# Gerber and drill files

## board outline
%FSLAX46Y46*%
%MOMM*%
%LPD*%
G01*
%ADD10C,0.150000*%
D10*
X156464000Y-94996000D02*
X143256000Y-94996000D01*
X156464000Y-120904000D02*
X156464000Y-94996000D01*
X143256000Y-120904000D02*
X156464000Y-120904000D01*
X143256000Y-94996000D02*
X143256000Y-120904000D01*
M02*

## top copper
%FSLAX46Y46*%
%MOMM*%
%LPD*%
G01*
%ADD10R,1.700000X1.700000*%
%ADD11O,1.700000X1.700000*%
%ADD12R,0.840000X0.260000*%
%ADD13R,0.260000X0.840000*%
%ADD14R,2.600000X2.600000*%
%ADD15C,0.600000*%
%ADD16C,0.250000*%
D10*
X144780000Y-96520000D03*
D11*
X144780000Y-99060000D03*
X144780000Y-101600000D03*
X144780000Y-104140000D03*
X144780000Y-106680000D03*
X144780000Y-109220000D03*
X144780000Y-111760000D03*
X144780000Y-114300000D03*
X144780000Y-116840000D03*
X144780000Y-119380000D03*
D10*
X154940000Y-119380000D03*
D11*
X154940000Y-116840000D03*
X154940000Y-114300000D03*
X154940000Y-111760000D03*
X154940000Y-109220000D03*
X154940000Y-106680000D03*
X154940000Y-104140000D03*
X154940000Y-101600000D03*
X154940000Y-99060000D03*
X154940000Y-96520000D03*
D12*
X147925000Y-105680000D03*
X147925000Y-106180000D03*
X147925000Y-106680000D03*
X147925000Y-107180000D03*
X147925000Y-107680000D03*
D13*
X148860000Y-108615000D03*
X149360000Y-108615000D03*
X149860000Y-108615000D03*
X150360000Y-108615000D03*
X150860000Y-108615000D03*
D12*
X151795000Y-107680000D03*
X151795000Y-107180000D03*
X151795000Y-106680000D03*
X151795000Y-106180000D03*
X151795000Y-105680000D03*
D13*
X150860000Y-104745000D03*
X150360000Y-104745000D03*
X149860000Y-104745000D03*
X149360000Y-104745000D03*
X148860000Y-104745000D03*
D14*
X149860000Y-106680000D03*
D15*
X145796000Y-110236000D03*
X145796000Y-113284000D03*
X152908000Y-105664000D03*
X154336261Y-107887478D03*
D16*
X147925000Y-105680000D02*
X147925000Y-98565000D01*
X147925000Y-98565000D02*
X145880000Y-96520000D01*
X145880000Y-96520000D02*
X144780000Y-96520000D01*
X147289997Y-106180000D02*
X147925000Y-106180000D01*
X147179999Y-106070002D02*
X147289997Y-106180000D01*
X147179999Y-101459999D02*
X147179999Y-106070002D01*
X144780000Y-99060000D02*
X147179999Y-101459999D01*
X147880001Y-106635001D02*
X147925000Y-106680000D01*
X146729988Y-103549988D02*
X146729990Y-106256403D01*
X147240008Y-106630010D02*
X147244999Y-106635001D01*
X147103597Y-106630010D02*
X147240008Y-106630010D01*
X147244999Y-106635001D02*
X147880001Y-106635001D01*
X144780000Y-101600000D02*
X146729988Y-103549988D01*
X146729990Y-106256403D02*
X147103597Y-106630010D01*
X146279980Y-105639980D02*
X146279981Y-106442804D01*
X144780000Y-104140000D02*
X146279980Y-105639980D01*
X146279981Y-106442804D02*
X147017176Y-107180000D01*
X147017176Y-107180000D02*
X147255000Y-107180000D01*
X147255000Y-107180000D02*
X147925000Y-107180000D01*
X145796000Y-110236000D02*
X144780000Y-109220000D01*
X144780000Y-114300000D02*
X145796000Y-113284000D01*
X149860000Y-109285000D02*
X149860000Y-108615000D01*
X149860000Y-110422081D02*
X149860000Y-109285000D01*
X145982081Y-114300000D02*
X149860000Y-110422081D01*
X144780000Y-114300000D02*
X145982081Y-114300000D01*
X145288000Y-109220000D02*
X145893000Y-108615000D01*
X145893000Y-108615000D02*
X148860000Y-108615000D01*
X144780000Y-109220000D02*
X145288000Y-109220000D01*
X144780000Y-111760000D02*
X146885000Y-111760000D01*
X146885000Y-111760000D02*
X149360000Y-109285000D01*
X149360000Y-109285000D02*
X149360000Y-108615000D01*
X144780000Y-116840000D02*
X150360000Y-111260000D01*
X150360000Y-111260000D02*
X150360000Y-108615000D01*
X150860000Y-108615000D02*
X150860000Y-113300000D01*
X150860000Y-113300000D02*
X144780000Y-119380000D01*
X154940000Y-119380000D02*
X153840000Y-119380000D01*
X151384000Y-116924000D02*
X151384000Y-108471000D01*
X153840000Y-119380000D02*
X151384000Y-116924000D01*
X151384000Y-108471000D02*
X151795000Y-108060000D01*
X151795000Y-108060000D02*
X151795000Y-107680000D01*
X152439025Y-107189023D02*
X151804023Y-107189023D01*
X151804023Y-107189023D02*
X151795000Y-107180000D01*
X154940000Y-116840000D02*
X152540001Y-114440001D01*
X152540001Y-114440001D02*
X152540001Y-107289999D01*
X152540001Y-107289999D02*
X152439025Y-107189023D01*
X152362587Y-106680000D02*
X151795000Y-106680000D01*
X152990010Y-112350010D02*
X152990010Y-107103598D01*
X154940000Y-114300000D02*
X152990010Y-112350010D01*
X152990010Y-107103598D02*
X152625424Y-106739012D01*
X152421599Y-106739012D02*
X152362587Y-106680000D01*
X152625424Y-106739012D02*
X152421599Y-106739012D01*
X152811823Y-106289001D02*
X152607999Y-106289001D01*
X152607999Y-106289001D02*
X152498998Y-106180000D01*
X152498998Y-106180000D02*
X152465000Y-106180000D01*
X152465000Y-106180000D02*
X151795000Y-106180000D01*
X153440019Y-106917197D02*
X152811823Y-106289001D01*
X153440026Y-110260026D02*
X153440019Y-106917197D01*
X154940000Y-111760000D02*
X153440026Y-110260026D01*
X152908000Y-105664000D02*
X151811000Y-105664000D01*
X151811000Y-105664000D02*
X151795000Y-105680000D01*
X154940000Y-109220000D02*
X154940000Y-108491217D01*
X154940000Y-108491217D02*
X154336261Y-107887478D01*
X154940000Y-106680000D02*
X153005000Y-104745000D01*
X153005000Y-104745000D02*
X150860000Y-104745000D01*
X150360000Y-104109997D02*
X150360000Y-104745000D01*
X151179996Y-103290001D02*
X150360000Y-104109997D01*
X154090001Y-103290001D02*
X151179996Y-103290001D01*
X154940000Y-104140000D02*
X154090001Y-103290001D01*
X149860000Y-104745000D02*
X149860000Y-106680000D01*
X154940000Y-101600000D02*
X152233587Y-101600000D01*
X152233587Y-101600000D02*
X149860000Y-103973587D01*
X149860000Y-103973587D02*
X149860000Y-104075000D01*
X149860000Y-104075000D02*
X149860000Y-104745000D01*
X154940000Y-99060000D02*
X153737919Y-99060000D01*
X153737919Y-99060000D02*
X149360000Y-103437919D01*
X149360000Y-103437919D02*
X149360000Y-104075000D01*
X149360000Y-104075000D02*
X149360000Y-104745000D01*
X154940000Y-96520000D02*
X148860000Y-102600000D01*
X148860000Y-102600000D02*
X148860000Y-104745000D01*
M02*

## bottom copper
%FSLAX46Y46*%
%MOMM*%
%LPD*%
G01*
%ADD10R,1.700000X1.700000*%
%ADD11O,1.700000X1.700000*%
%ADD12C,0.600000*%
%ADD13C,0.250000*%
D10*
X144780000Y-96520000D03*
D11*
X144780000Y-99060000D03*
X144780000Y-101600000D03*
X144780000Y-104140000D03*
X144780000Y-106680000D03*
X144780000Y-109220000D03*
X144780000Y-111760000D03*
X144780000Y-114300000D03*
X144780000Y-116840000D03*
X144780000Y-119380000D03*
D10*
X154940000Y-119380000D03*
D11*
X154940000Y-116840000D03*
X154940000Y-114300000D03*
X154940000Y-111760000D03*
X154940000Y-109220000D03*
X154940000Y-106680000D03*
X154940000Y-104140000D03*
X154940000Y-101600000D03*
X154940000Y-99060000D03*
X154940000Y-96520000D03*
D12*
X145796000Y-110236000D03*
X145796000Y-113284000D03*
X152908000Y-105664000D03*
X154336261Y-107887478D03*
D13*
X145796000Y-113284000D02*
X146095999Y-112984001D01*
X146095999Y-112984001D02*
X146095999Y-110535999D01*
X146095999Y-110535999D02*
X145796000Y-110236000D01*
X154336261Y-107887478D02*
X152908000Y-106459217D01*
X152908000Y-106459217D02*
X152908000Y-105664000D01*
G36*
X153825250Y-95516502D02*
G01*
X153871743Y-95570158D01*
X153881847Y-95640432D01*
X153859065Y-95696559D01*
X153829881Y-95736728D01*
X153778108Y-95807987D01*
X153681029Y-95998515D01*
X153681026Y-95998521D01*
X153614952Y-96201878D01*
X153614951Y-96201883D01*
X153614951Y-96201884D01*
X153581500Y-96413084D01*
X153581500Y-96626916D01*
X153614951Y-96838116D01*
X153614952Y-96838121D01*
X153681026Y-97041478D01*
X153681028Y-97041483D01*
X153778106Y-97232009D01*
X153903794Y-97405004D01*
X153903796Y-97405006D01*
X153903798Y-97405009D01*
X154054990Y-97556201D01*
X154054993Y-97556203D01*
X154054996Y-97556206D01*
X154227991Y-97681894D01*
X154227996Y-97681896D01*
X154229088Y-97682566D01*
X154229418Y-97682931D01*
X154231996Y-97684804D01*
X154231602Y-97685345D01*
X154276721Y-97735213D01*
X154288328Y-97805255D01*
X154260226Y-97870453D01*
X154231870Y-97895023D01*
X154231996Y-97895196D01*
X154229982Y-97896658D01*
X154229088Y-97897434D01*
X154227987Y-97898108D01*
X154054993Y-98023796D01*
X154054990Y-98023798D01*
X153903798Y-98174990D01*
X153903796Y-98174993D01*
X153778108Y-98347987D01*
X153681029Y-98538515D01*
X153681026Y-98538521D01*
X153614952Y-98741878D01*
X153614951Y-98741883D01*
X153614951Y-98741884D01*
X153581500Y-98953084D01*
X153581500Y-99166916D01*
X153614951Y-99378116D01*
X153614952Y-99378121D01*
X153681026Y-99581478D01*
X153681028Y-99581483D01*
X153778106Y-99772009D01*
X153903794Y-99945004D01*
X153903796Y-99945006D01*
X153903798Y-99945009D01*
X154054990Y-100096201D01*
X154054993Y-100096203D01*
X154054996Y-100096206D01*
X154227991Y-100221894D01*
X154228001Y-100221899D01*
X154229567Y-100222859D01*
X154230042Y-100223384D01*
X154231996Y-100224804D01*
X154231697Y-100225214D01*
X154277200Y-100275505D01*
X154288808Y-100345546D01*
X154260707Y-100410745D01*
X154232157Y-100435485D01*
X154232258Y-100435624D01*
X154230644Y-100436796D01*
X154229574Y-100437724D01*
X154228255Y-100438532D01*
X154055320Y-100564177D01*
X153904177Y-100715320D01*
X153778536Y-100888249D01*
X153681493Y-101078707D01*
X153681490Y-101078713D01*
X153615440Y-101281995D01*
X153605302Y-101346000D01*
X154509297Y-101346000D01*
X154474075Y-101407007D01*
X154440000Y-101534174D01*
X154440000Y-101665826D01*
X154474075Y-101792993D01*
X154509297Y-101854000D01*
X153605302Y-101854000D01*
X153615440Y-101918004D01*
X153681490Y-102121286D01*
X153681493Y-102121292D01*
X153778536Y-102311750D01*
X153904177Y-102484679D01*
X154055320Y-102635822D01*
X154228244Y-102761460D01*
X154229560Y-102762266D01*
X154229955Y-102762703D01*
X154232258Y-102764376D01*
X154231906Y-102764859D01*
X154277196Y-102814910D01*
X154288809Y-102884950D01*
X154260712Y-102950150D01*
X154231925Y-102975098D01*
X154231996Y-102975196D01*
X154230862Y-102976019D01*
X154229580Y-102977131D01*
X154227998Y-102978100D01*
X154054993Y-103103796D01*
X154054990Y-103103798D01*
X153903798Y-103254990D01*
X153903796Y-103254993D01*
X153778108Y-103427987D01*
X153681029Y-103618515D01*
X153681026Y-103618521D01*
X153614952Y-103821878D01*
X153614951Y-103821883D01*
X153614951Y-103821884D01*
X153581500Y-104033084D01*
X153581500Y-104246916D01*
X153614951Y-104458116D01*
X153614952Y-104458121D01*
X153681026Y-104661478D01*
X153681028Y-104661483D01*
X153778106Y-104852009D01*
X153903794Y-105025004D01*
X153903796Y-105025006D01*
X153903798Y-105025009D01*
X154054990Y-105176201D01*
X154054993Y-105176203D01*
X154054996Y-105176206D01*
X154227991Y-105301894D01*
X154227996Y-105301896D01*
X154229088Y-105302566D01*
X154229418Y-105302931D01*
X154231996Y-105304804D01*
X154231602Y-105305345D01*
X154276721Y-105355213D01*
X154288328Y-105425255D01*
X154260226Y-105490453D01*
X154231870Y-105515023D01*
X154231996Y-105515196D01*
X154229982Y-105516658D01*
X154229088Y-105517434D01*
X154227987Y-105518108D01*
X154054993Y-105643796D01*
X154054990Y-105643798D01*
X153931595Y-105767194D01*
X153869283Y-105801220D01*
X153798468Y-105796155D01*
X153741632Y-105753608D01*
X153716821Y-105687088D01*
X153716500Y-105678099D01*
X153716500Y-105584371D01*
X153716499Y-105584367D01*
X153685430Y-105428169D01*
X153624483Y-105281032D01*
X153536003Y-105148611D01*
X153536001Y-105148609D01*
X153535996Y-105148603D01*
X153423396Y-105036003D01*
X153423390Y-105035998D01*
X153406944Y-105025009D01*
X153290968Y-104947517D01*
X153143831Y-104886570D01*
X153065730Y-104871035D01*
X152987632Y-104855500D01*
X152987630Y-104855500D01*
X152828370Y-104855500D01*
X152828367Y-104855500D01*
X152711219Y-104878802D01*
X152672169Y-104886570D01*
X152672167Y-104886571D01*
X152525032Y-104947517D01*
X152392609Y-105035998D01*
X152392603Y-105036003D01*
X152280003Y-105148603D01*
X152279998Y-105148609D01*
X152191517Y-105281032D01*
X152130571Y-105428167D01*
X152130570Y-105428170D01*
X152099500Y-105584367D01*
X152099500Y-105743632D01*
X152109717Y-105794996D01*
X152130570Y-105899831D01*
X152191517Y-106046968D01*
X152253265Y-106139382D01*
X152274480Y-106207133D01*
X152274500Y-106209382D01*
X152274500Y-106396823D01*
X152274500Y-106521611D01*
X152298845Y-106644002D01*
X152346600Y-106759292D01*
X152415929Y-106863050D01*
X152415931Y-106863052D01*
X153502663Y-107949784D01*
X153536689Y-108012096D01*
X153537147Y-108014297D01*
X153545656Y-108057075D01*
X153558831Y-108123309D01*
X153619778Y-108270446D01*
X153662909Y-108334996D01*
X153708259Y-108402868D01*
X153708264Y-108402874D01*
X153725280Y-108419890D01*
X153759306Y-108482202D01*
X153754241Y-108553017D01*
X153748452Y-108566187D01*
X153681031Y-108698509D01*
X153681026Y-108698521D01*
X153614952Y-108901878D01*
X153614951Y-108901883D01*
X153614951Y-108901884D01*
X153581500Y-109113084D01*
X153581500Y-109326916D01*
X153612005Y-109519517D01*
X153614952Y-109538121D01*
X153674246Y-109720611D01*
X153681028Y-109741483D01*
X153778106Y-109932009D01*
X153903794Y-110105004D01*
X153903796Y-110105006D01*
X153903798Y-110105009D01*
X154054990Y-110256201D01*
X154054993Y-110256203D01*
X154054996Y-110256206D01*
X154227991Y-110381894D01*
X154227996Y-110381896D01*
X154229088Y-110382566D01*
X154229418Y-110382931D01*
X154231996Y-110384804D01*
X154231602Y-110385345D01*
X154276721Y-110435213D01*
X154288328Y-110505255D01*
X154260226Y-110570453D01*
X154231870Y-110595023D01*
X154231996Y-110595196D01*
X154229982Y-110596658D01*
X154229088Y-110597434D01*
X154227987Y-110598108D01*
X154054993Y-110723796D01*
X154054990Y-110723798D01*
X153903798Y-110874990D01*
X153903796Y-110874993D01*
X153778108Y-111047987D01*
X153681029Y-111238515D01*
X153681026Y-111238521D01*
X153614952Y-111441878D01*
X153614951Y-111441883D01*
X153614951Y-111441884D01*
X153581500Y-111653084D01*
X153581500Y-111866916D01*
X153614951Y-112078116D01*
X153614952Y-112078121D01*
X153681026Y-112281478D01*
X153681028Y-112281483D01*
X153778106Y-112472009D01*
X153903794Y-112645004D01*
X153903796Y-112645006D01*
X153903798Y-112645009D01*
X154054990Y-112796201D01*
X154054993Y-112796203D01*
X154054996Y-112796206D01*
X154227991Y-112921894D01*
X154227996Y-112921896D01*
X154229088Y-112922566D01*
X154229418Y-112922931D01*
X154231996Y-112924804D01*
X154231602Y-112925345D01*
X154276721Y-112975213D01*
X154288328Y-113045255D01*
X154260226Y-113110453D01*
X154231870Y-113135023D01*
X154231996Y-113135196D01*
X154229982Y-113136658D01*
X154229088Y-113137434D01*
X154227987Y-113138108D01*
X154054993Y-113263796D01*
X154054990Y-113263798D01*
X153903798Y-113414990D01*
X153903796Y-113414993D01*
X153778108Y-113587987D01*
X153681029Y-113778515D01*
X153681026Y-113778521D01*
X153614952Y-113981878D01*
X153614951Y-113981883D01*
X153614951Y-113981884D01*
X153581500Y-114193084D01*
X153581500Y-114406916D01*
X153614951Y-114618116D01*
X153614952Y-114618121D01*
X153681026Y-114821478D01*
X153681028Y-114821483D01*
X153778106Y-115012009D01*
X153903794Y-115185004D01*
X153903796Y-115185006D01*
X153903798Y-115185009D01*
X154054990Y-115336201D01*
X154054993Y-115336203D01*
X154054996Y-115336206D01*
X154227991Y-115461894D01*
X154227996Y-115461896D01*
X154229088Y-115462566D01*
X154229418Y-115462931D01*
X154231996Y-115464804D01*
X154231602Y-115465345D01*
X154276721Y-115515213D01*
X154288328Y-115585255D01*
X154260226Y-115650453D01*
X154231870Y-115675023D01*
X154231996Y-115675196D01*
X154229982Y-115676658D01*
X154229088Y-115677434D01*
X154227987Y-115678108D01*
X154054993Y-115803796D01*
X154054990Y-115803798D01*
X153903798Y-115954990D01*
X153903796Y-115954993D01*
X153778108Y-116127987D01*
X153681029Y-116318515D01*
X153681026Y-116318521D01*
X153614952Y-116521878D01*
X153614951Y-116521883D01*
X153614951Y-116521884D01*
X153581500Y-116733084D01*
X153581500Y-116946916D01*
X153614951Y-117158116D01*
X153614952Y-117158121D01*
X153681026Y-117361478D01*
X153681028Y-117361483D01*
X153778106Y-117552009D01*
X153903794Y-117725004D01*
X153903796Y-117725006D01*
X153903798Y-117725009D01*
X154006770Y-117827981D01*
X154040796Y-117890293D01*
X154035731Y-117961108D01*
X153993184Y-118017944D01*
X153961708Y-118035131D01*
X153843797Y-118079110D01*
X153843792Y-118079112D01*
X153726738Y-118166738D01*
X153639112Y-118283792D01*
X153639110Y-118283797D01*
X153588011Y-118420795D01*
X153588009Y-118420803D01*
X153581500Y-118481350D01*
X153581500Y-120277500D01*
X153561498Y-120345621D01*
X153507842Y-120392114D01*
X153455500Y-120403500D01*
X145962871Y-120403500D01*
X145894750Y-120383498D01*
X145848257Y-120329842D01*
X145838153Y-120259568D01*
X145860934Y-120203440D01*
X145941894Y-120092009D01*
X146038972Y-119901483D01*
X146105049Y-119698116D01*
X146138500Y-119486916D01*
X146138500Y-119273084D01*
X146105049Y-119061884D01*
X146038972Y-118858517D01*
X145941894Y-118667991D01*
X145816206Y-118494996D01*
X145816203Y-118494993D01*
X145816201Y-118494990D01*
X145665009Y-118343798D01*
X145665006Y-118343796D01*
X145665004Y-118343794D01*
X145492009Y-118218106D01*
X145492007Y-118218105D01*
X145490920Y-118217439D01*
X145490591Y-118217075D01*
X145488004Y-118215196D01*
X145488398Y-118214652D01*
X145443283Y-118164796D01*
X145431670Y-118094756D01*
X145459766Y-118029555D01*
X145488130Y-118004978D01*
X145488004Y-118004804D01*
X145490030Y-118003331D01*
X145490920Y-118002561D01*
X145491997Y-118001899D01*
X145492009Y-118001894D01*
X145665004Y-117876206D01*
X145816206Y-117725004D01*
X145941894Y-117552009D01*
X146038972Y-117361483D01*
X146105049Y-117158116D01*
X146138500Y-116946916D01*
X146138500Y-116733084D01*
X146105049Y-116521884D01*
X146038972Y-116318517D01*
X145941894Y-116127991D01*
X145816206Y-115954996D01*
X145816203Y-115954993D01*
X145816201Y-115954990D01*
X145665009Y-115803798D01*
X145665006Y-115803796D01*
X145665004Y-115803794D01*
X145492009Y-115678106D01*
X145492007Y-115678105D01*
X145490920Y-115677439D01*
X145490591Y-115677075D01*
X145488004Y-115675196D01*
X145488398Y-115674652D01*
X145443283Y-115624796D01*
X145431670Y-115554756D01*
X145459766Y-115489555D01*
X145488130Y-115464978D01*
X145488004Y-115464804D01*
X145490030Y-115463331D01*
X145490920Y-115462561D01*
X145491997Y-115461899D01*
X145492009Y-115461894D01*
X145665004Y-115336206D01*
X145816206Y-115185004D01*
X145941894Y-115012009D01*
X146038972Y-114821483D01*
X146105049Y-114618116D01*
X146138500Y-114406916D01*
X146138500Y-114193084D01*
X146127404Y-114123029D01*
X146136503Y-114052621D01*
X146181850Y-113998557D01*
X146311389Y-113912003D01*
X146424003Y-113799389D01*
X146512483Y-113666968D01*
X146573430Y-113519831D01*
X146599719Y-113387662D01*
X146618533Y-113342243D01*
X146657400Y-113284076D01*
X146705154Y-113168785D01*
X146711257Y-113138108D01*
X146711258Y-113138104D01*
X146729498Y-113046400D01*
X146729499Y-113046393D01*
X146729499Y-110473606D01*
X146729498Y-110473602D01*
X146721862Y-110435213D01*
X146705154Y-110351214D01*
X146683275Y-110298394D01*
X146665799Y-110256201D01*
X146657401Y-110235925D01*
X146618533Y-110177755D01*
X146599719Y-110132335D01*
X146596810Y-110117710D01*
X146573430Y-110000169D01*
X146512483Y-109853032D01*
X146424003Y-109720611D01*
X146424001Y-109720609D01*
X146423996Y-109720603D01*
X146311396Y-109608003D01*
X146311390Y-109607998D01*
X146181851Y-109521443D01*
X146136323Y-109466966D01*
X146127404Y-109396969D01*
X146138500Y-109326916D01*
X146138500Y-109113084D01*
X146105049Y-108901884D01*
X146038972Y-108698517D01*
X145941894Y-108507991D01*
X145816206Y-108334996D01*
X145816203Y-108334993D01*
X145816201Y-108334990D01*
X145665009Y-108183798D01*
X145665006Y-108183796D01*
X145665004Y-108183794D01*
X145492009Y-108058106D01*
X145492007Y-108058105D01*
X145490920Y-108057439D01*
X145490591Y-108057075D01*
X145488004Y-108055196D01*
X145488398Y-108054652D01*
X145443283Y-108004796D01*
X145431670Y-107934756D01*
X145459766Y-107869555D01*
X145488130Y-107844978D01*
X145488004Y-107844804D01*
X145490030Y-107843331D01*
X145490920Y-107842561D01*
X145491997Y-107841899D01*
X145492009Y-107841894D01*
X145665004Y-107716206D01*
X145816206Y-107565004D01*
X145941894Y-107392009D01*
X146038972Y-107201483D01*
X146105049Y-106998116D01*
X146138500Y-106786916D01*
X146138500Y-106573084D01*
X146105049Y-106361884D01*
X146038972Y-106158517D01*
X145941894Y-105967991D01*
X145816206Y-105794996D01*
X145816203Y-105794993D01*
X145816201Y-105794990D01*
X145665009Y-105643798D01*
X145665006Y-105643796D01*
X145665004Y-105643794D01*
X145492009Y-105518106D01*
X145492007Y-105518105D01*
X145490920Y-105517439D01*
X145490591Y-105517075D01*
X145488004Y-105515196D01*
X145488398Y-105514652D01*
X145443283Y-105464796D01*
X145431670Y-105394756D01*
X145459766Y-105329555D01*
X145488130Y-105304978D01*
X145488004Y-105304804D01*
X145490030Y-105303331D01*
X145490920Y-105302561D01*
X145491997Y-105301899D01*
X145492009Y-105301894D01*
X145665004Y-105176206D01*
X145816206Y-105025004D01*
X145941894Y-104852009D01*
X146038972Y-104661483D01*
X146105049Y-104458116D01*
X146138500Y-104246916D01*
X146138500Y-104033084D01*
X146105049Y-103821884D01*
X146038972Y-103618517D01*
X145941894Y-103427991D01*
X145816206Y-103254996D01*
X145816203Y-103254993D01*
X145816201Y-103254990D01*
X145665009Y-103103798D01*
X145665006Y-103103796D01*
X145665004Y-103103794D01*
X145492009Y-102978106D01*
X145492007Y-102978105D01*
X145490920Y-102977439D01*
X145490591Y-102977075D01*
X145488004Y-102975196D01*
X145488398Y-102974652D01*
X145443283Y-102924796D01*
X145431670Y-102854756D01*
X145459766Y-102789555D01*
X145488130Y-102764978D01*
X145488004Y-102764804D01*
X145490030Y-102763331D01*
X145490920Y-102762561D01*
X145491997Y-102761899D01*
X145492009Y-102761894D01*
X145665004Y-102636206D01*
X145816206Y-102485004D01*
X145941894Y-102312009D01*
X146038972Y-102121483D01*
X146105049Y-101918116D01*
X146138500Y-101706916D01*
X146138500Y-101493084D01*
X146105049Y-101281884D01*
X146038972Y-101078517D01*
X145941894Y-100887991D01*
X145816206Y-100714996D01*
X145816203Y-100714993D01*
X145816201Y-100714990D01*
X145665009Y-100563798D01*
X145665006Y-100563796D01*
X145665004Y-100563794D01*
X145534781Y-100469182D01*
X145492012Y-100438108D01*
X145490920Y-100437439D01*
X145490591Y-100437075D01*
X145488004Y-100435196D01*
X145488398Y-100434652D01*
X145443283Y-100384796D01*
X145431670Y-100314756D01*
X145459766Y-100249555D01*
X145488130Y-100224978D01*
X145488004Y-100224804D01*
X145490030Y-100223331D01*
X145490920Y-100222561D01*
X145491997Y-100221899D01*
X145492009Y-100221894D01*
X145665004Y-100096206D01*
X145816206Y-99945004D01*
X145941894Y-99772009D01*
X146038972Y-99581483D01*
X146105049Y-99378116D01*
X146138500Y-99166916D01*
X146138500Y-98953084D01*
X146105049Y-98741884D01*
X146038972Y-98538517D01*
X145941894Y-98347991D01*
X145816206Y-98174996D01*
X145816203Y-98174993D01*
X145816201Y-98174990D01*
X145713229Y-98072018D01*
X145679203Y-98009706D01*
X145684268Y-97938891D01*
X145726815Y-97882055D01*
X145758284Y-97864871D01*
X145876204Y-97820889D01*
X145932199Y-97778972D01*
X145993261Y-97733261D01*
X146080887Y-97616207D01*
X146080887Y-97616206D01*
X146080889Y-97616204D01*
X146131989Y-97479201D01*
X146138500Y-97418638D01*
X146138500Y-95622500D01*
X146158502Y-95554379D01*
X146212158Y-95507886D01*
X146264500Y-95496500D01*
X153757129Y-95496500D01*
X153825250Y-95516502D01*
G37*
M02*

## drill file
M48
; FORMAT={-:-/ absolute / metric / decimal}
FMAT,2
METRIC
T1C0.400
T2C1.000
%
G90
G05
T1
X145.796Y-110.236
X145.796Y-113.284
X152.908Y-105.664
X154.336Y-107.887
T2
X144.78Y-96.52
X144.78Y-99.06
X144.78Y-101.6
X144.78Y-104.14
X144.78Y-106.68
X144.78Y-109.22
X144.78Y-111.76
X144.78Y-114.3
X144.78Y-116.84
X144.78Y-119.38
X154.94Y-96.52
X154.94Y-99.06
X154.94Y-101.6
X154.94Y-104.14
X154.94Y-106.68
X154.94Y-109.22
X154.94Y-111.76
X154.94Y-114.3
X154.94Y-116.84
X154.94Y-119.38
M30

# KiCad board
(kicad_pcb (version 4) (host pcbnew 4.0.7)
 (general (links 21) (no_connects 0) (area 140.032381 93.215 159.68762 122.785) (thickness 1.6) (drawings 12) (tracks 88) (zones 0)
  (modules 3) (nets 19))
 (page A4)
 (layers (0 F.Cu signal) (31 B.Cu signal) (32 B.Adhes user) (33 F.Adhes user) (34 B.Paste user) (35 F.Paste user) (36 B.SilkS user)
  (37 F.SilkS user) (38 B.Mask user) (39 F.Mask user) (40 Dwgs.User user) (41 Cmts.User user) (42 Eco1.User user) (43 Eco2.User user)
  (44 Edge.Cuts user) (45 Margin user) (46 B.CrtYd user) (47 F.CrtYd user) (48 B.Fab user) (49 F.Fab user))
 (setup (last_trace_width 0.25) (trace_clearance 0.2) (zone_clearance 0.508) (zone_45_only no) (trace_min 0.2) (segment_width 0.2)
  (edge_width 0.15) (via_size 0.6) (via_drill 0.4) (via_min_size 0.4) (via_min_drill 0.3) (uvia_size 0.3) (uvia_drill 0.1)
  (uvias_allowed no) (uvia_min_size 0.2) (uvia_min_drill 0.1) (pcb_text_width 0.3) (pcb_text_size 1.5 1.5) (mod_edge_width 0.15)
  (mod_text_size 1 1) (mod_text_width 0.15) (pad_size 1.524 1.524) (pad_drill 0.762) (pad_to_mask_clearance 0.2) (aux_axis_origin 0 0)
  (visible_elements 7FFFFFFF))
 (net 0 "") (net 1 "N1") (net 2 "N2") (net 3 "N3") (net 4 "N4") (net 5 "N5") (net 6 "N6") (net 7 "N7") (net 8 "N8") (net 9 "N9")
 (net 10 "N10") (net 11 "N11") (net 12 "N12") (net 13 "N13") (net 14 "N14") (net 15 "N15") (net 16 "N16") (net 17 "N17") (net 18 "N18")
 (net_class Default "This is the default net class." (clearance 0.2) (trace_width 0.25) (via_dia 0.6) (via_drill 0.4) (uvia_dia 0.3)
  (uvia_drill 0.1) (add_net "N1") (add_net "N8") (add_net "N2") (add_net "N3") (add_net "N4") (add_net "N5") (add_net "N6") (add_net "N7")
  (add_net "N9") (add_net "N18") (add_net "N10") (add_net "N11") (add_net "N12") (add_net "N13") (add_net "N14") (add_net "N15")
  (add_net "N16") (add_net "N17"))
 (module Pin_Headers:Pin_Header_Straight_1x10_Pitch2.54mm (layer F.Cu) (at 144.78 96.52)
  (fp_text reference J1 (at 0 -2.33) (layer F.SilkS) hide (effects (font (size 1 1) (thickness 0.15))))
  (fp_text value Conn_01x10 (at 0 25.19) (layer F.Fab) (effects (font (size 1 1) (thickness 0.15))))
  (pad 1 thru_hole rect (at 0 0) (size 1.7 1.7) (drill 1) (layers *.Cu *.Mask) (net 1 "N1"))
  (pad 2 thru_hole oval (at 0 2.54) (size 1.7 1.7) (drill 1) (layers *.Cu *.Mask) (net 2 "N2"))
  (pad 3 thru_hole oval (at 0 5.08) (size 1.7 1.7) (drill 1) (layers *.Cu *.Mask) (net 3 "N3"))
  (pad 4 thru_hole oval (at 0 7.62) (size 1.7 1.7) (drill 1) (layers *.Cu *.Mask) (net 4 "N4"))
  (pad 5 thru_hole oval (at 0 10.16) (size 1.7 1.7) (drill 1) (layers *.Cu *.Mask))
  (pad 6 thru_hole oval (at 0 12.7) (size 1.7 1.7) (drill 1) (layers *.Cu *.Mask) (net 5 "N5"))
  (pad 7 thru_hole oval (at 0 15.24) (size 1.7 1.7) (drill 1) (layers *.Cu *.Mask) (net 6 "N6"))
  (pad 8 thru_hole oval (at 0 17.78) (size 1.7 1.7) (drill 1) (layers *.Cu *.Mask) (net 5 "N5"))
  (pad 9 thru_hole oval (at 0 20.32) (size 1.7 1.7) (drill 1) (layers *.Cu *.Mask) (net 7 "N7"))
  (pad 10 thru_hole oval (at 0 22.86) (size 1.7 1.7) (drill 1) (layers *.Cu *.Mask) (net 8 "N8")))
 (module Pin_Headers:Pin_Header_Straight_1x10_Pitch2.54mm (layer F.Cu) (at 154.94 119.38 180)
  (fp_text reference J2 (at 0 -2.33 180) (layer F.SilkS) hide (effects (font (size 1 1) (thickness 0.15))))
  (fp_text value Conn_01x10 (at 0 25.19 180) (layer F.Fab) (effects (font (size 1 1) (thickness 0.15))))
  (pad 1 thru_hole rect (at 0 0 180) (size 1.7 1.7) (drill 1) (layers *.Cu *.Mask) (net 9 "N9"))
  (pad 2 thru_hole oval (at 0 2.54 180) (size 1.7 1.7) (drill 1) (layers *.Cu *.Mask) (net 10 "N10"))
  (pad 3 thru_hole oval (at 0 5.08 180) (size 1.7 1.7) (drill 1) (layers *.Cu *.Mask) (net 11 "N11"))
  (pad 4 thru_hole oval (at 0 7.62 180) (size 1.7 1.7) (drill 1) (layers *.Cu *.Mask) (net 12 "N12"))
  (pad 5 thru_hole oval (at 0 10.16 180) (size 1.7 1.7) (drill 1) (layers *.Cu *.Mask) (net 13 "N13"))
  (pad 6 thru_hole oval (at 0 12.7 180) (size 1.7 1.7) (drill 1) (layers *.Cu *.Mask) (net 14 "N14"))
  (pad 7 thru_hole oval (at 0 15.24 180) (size 1.7 1.7) (drill 1) (layers *.Cu *.Mask) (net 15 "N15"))
  (pad 8 thru_hole oval (at 0 17.78 180) (size 1.7 1.7) (drill 1) (layers *.Cu *.Mask) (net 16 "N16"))
  (pad 9 thru_hole oval (at 0 20.32 180) (size 1.7 1.7) (drill 1) (layers *.Cu *.Mask) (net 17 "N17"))
  (pad 10 thru_hole oval (at 0 22.86 180) (size 1.7 1.7) (drill 1) (layers *.Cu *.Mask) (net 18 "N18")))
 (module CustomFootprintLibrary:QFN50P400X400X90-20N (layer F.Cu) (at 149.86 106.68)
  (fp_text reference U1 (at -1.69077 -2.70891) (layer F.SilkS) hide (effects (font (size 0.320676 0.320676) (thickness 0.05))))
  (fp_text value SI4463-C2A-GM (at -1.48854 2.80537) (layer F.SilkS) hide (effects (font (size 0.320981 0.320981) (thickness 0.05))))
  (pad 1 smd rect (at -1.935 -1 90) (size 0.26 0.84) (layers F.Cu F.Paste F.Mask) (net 1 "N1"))
  (pad 2 smd rect (at -1.935 -0.5 90) (size 0.26 0.84) (layers F.Cu F.Paste F.Mask) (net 2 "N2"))
  (pad 3 smd rect (at -1.935 0 90) (size 0.26 0.84) (layers F.Cu F.Paste F.Mask) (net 3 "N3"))
  (pad 4 smd rect (at -1.935 0.5 90) (size 0.26 0.84) (layers F.Cu F.Paste F.Mask) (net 4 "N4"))
  (pad 5 smd rect (at -1.935 1 90) (size 0.26 0.84) (layers F.Cu F.Paste F.Mask))
  (pad 6 smd rect (at -1 1.935 180) (size 0.26 0.84) (layers F.Cu F.Paste F.Mask) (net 5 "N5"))
  (pad 7 smd rect (at -0.5 1.935 180) (size 0.26 0.84) (layers F.Cu F.Paste F.Mask) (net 6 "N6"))
  (pad 8 smd rect (at 0 1.935 180) (size 0.26 0.84) (layers F.Cu F.Paste F.Mask) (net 5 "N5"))
  (pad 9 smd rect (at 0.5 1.935 180) (size 0.26 0.84) (layers F.Cu F.Paste F.Mask) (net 7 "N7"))
  (pad 10 smd rect (at 1 1.935 180) (size 0.26 0.84) (layers F.Cu F.Paste F.Mask) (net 8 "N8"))
  (pad 11 smd rect (at 1.935 1 270) (size 0.26 0.84) (layers F.Cu F.Paste F.Mask) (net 9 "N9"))
  (pad 12 smd rect (at 1.935 0.5 270) (size 0.26 0.84) (layers F.Cu F.Paste F.Mask) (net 10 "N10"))
  (pad 13 smd rect (at 1.935 0 270) (size 0.26 0.84) (layers F.Cu F.Paste F.Mask) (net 11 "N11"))
  (pad 14 smd rect (at 1.935 -0.5 270) (size 0.26 0.84) (layers F.Cu F.Paste F.Mask) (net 12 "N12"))
  (pad 15 smd rect (at 1.935 -1 270) (size 0.26 0.84) (layers F.Cu F.Paste F.Mask) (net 13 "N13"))
  (pad 16 smd rect (at 1 -1.935) (size 0.26 0.84) (layers F.Cu F.Paste F.Mask) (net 14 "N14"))
  (pad 17 smd rect (at 0.5 -1.935) (size 0.26 0.84) (layers F.Cu F.Paste F.Mask) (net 15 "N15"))
  (pad 18 smd rect (at 0 -1.935) (size 0.26 0.84) (layers F.Cu F.Paste F.Mask) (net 16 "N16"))
  (pad 19 smd rect (at -0.5 -1.935) (size 0.26 0.84) (layers F.Cu F.Paste F.Mask) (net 17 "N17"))
  (pad 20 smd rect (at -1 -1.935) (size 0.26 0.84) (layers F.Cu F.Paste F.Mask) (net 18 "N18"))
  (pad 21 smd rect (at 0 0) (size 2.6 2.6) (layers F.Cu F.Paste F.Mask) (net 16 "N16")))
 (gr_line (start 156.464 94.996) (end 143.256 94.996) (layer Edge.Cuts) (width 0.15))
 (gr_line (start 156.464 120.904) (end 156.464 94.996) (layer Edge.Cuts) (width 0.15))
 (gr_line (start 143.256 120.904) (end 156.464 120.904) (layer Edge.Cuts) (width 0.15))
 (gr_line (start 143.256 94.996) (end 143.256 120.904) (layer Edge.Cuts) (width 0.15))
 (segment (start 147.925 105.68) (end 147.925 98.565) (width 0.25) (layer F.Cu) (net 1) (status 10))
 (segment (start 147.925 98.565) (end 145.88 96.52) (width 0.25) (layer F.Cu) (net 1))
 (segment (start 145.88 96.52) (end 144.78 96.52) (width 0.25) (layer F.Cu) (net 1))
 (segment (start 147.289997 106.18) (end 147.925 106.18) (width 0.25) (layer F.Cu) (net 2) (status 20))
 (segment (start 147.179999 106.070002) (end 147.289997 106.18) (width 0.25) (layer F.Cu) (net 2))
 (segment (start 147.179999 101.459999) (end 147.179999 106.070002) (width 0.25) (layer F.Cu) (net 2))
 (segment (start 144.78 99.06) (end 147.179999 101.459999) (width 0.25) (layer F.Cu) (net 2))
 (segment (start 147.880001 106.635001) (end 147.925 106.68) (width 0.25) (layer F.Cu) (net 3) (status 30))
 (segment (start 146.729988 103.549988) (end 146.72999 106.256403) (width 0.25) (layer F.Cu) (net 3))
 (segment (start 147.240008 106.63001) (end 147.244999 106.635001) (width 0.25) (layer F.Cu) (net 3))
 (segment (start 147.103597 106.63001) (end 147.240008 106.63001) (width 0.25) (layer F.Cu) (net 3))
 (segment (start 147.244999 106.635001) (end 147.880001 106.635001) (width 0.25) (layer F.Cu) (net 3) (status 20))
 (segment (start 144.78 101.6) (end 146.729988 103.549988) (width 0.25) (layer F.Cu) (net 3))
 (segment (start 146.72999 106.256403) (end 147.103597 106.63001) (width 0.25) (layer F.Cu) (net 3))
 (segment (start 146.27998 105.63998) (end 146.279981 106.442804) (width 0.25) (layer F.Cu) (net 4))
 (segment (start 144.78 104.14) (end 146.27998 105.63998) (width 0.25) (layer F.Cu) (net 4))
 (segment (start 146.279981 106.442804) (end 147.017176 107.18) (width 0.25) (layer F.Cu) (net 4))
 (segment (start 147.017176 107.18) (end 147.255 107.18) (width 0.25) (layer F.Cu) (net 4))
 (segment (start 147.255 107.18) (end 147.925 107.18) (width 0.25) (layer F.Cu) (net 4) (status 20))
 (segment (start 145.796 110.236) (end 144.78 109.22) (width 0.25) (layer F.Cu) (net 5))
 (segment (start 145.796 113.284) (end 146.095999 112.984001) (width 0.25) (layer B.Cu) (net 5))
 (segment (start 146.095999 112.984001) (end 146.095999 110.535999) (width 0.25) (layer B.Cu) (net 5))
 (segment (start 146.095999 110.535999) (end 145.796 110.236) (width 0.25) (layer B.Cu) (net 5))
 (via (at 145.796 110.236) (size 0.6) (drill 0.4) (layers F.Cu B.Cu) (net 5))
 (segment (start 144.78 114.3) (end 145.796 113.284) (width 0.25) (layer F.Cu) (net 5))
 (via (at 145.796 113.284) (size 0.6) (drill 0.4) (layers F.Cu B.Cu) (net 5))
 (segment (start 149.86 109.285) (end 149.86 108.615) (width 0.25) (layer F.Cu) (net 5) (status 20))
 (segment (start 149.86 110.422081) (end 149.86 109.285) (width 0.25) (layer F.Cu) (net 5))
 (segment (start 145.982081 114.3) (end 149.86 110.422081) (width 0.25) (layer F.Cu) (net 5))
 (segment (start 144.78 114.3) (end 145.982081 114.3) (width 0.25) (layer F.Cu) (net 5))
 (segment (start 145.288 109.22) (end 145.893 108.615) (width 0.25) (layer F.Cu) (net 5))
 (segment (start 145.893 108.615) (end 148.86 108.615) (width 0.25) (layer F.Cu) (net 5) (status 20))
 (segment (start 144.78 109.22) (end 145.288 109.22) (width 0.25) (layer F.Cu) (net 5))
 (segment (start 144.78 111.76) (end 146.885 111.76) (width 0.25) (layer F.Cu) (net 6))
 (segment (start 146.885 111.76) (end 149.36 109.285) (width 0.25) (layer F.Cu) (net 6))
 (segment (start 149.36 109.285) (end 149.36 108.615) (width 0.25) (layer F.Cu) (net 6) (status 20))
 (segment (start 144.78 116.84) (end 150.36 111.26) (width 0.25) (layer F.Cu) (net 7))
 (segment (start 150.36 111.26) (end 150.36 108.615) (width 0.25) (layer F.Cu) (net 7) (status 20))
 (segment (start 150.86 108.615) (end 150.86 113.3) (width 0.25) (layer F.Cu) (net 8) (status 10))
 (segment (start 150.86 113.3) (end 144.78 119.38) (width 0.25) (layer F.Cu) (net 8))
 (segment (start 154.94 119.38) (end 153.84 119.38) (width 0.25) (layer F.Cu) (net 9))
 (segment (start 151.384 116.924) (end 151.384 108.471) (width 0.25) (layer F.Cu) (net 9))
 (segment (start 153.84 119.38) (end 151.384 116.924) (width 0.25) (layer F.Cu) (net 9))
 (segment (start 151.384 108.471) (end 151.795 108.06) (width 0.25) (layer F.Cu) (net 9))
 (segment (start 151.795 108.06) (end 151.795 107.68) (width 0.25) (layer F.Cu) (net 9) (status 20))
 (segment (start 152.439025 107.189023) (end 151.804023 107.189023) (width 0.25) (layer F.Cu) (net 10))
 (segment (start 151.804023 107.189023) (end 151.795 107.18) (width 0.25) (layer F.Cu) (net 10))
 (segment (start 154.94 116.84) (end 152.540001 114.440001) (width 0.25) (layer F.Cu) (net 10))
 (segment (start 152.540001 114.440001) (end 152.540001 107.289999) (width 0.25) (layer F.Cu) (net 10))
 (segment (start 152.540001 107.289999) (end 152.439025 107.189023) (width 0.25) (layer F.Cu) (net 10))
 (segment (start 152.362587 106.68) (end 151.795 106.68) (width 0.25) (layer F.Cu) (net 11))
 (segment (start 152.99001 112.35001) (end 152.99001 107.103598) (width 0.25) (layer F.Cu) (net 11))
 (segment (start 154.94 114.3) (end 152.99001 112.35001) (width 0.25) (layer F.Cu) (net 11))
 (segment (start 152.99001 107.103598) (end 152.625424 106.739012) (width 0.25) (layer F.Cu) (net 11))
 (segment (start 152.421599 106.739012) (end 152.362587 106.68) (width 0.25) (layer F.Cu) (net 11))
 (segment (start 152.625424 106.739012) (end 152.421599 106.739012) (width 0.25) (layer F.Cu) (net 11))
 (segment (start 152.811823 106.289001) (end 152.607999 106.289001) (width 0.25) (layer F.Cu) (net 12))
 (segment (start 152.607999 106.289001) (end 152.498998 106.18) (width 0.25) (layer F.Cu) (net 12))
 (segment (start 152.498998 106.18) (end 152.465 106.18) (width 0.25) (layer F.Cu) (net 12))
 (segment (start 152.465 106.18) (end 151.795 106.18) (width 0.25) (layer F.Cu) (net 12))
 (segment (start 153.440019 106.917197) (end 152.811823 106.289001) (width 0.25) (layer F.Cu) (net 12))
 (segment (start 153.440026 110.260026) (end 153.440019 106.917197) (width 0.25) (layer F.Cu) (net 12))
 (segment (start 154.94 111.76) (end 153.440026 110.260026) (width 0.25) (layer F.Cu) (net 12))
 (segment (start 152.908 105.664) (end 151.811 105.664) (width 0.25) (layer F.Cu) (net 13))
 (segment (start 151.811 105.664) (end 151.795 105.68) (width 0.25) (layer F.Cu) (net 13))
 (segment (start 154.336261 107.887478) (end 152.908 106.459217) (width 0.25) (layer B.Cu) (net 13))
 (via (at 152.908 105.664) (size 0.6) (drill 0.4) (layers F.Cu B.Cu) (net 13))
 (segment (start 152.908 106.459217) (end 152.908 105.664) (width 0.25) (layer B.Cu) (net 13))
 (segment (start 154.94 109.22) (end 154.94 108.491217) (width 0.25) (layer F.Cu) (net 13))
 (segment (start 154.94 108.491217) (end 154.336261 107.887478) (width 0.25) (layer F.Cu) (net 13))
 (via (at 154.336261 107.887478) (size 0.6) (drill 0.4) (layers F.Cu B.Cu) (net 13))
 (segment (start 154.94 106.68) (end 153.005 104.745) (width 0.25) (layer F.Cu) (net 14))
 (segment (start 153.005 104.745) (end 150.86 104.745) (width 0.25) (layer F.Cu) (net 14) (status 20))
 (segment (start 150.36 104.109997) (end 150.36 104.745) (width 0.25) (layer F.Cu) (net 15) (status 20))
 (segment (start 151.179996 103.290001) (end 150.36 104.109997) (width 0.25) (layer F.Cu) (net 15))
 (segment (start 154.090001 103.290001) (end 151.179996 103.290001) (width 0.25) (layer F.Cu) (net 15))
 (segment (start 154.94 104.14) (end 154.090001 103.290001) (width 0.25) (layer F.Cu) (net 15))
 (segment (start 149.86 104.745) (end 149.86 106.68) (width 0.25) (layer F.Cu) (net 16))
 (segment (start 154.94 101.6) (end 152.233587 101.6) (width 0.25) (layer F.Cu) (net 16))
 (segment (start 152.233587 101.6) (end 149.86 103.973587) (width 0.25) (layer F.Cu) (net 16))
 (segment (start 149.86 103.973587) (end 149.86 104.075) (width 0.25) (layer F.Cu) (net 16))
 (segment (start 149.86 104.075) (end 149.86 104.745) (width 0.25) (layer F.Cu) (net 16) (status 20))
 (segment (start 154.94 99.06) (end 153.737919 99.06) (width 0.25) (layer F.Cu) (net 17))
 (segment (start 153.737919 99.06) (end 149.36 103.437919) (width 0.25) (layer F.Cu) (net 17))
 (segment (start 149.36 103.437919) (end 149.36 104.075) (width 0.25) (layer F.Cu) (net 17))
 (segment (start 149.36 104.075) (end 149.36 104.745) (width 0.25) (layer F.Cu) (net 17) (status 20))
 (segment (start 154.94 96.52) (end 148.86 102.6) (width 0.25) (layer F.Cu) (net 18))
 (segment (start 148.86 102.6) (end 148.86 104.745) (width 0.25) (layer F.Cu) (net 18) (status 20))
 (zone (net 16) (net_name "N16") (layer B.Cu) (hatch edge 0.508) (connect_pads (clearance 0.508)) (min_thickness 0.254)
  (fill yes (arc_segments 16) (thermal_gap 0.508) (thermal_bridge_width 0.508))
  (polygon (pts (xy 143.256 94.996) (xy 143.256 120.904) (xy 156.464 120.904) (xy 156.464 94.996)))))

